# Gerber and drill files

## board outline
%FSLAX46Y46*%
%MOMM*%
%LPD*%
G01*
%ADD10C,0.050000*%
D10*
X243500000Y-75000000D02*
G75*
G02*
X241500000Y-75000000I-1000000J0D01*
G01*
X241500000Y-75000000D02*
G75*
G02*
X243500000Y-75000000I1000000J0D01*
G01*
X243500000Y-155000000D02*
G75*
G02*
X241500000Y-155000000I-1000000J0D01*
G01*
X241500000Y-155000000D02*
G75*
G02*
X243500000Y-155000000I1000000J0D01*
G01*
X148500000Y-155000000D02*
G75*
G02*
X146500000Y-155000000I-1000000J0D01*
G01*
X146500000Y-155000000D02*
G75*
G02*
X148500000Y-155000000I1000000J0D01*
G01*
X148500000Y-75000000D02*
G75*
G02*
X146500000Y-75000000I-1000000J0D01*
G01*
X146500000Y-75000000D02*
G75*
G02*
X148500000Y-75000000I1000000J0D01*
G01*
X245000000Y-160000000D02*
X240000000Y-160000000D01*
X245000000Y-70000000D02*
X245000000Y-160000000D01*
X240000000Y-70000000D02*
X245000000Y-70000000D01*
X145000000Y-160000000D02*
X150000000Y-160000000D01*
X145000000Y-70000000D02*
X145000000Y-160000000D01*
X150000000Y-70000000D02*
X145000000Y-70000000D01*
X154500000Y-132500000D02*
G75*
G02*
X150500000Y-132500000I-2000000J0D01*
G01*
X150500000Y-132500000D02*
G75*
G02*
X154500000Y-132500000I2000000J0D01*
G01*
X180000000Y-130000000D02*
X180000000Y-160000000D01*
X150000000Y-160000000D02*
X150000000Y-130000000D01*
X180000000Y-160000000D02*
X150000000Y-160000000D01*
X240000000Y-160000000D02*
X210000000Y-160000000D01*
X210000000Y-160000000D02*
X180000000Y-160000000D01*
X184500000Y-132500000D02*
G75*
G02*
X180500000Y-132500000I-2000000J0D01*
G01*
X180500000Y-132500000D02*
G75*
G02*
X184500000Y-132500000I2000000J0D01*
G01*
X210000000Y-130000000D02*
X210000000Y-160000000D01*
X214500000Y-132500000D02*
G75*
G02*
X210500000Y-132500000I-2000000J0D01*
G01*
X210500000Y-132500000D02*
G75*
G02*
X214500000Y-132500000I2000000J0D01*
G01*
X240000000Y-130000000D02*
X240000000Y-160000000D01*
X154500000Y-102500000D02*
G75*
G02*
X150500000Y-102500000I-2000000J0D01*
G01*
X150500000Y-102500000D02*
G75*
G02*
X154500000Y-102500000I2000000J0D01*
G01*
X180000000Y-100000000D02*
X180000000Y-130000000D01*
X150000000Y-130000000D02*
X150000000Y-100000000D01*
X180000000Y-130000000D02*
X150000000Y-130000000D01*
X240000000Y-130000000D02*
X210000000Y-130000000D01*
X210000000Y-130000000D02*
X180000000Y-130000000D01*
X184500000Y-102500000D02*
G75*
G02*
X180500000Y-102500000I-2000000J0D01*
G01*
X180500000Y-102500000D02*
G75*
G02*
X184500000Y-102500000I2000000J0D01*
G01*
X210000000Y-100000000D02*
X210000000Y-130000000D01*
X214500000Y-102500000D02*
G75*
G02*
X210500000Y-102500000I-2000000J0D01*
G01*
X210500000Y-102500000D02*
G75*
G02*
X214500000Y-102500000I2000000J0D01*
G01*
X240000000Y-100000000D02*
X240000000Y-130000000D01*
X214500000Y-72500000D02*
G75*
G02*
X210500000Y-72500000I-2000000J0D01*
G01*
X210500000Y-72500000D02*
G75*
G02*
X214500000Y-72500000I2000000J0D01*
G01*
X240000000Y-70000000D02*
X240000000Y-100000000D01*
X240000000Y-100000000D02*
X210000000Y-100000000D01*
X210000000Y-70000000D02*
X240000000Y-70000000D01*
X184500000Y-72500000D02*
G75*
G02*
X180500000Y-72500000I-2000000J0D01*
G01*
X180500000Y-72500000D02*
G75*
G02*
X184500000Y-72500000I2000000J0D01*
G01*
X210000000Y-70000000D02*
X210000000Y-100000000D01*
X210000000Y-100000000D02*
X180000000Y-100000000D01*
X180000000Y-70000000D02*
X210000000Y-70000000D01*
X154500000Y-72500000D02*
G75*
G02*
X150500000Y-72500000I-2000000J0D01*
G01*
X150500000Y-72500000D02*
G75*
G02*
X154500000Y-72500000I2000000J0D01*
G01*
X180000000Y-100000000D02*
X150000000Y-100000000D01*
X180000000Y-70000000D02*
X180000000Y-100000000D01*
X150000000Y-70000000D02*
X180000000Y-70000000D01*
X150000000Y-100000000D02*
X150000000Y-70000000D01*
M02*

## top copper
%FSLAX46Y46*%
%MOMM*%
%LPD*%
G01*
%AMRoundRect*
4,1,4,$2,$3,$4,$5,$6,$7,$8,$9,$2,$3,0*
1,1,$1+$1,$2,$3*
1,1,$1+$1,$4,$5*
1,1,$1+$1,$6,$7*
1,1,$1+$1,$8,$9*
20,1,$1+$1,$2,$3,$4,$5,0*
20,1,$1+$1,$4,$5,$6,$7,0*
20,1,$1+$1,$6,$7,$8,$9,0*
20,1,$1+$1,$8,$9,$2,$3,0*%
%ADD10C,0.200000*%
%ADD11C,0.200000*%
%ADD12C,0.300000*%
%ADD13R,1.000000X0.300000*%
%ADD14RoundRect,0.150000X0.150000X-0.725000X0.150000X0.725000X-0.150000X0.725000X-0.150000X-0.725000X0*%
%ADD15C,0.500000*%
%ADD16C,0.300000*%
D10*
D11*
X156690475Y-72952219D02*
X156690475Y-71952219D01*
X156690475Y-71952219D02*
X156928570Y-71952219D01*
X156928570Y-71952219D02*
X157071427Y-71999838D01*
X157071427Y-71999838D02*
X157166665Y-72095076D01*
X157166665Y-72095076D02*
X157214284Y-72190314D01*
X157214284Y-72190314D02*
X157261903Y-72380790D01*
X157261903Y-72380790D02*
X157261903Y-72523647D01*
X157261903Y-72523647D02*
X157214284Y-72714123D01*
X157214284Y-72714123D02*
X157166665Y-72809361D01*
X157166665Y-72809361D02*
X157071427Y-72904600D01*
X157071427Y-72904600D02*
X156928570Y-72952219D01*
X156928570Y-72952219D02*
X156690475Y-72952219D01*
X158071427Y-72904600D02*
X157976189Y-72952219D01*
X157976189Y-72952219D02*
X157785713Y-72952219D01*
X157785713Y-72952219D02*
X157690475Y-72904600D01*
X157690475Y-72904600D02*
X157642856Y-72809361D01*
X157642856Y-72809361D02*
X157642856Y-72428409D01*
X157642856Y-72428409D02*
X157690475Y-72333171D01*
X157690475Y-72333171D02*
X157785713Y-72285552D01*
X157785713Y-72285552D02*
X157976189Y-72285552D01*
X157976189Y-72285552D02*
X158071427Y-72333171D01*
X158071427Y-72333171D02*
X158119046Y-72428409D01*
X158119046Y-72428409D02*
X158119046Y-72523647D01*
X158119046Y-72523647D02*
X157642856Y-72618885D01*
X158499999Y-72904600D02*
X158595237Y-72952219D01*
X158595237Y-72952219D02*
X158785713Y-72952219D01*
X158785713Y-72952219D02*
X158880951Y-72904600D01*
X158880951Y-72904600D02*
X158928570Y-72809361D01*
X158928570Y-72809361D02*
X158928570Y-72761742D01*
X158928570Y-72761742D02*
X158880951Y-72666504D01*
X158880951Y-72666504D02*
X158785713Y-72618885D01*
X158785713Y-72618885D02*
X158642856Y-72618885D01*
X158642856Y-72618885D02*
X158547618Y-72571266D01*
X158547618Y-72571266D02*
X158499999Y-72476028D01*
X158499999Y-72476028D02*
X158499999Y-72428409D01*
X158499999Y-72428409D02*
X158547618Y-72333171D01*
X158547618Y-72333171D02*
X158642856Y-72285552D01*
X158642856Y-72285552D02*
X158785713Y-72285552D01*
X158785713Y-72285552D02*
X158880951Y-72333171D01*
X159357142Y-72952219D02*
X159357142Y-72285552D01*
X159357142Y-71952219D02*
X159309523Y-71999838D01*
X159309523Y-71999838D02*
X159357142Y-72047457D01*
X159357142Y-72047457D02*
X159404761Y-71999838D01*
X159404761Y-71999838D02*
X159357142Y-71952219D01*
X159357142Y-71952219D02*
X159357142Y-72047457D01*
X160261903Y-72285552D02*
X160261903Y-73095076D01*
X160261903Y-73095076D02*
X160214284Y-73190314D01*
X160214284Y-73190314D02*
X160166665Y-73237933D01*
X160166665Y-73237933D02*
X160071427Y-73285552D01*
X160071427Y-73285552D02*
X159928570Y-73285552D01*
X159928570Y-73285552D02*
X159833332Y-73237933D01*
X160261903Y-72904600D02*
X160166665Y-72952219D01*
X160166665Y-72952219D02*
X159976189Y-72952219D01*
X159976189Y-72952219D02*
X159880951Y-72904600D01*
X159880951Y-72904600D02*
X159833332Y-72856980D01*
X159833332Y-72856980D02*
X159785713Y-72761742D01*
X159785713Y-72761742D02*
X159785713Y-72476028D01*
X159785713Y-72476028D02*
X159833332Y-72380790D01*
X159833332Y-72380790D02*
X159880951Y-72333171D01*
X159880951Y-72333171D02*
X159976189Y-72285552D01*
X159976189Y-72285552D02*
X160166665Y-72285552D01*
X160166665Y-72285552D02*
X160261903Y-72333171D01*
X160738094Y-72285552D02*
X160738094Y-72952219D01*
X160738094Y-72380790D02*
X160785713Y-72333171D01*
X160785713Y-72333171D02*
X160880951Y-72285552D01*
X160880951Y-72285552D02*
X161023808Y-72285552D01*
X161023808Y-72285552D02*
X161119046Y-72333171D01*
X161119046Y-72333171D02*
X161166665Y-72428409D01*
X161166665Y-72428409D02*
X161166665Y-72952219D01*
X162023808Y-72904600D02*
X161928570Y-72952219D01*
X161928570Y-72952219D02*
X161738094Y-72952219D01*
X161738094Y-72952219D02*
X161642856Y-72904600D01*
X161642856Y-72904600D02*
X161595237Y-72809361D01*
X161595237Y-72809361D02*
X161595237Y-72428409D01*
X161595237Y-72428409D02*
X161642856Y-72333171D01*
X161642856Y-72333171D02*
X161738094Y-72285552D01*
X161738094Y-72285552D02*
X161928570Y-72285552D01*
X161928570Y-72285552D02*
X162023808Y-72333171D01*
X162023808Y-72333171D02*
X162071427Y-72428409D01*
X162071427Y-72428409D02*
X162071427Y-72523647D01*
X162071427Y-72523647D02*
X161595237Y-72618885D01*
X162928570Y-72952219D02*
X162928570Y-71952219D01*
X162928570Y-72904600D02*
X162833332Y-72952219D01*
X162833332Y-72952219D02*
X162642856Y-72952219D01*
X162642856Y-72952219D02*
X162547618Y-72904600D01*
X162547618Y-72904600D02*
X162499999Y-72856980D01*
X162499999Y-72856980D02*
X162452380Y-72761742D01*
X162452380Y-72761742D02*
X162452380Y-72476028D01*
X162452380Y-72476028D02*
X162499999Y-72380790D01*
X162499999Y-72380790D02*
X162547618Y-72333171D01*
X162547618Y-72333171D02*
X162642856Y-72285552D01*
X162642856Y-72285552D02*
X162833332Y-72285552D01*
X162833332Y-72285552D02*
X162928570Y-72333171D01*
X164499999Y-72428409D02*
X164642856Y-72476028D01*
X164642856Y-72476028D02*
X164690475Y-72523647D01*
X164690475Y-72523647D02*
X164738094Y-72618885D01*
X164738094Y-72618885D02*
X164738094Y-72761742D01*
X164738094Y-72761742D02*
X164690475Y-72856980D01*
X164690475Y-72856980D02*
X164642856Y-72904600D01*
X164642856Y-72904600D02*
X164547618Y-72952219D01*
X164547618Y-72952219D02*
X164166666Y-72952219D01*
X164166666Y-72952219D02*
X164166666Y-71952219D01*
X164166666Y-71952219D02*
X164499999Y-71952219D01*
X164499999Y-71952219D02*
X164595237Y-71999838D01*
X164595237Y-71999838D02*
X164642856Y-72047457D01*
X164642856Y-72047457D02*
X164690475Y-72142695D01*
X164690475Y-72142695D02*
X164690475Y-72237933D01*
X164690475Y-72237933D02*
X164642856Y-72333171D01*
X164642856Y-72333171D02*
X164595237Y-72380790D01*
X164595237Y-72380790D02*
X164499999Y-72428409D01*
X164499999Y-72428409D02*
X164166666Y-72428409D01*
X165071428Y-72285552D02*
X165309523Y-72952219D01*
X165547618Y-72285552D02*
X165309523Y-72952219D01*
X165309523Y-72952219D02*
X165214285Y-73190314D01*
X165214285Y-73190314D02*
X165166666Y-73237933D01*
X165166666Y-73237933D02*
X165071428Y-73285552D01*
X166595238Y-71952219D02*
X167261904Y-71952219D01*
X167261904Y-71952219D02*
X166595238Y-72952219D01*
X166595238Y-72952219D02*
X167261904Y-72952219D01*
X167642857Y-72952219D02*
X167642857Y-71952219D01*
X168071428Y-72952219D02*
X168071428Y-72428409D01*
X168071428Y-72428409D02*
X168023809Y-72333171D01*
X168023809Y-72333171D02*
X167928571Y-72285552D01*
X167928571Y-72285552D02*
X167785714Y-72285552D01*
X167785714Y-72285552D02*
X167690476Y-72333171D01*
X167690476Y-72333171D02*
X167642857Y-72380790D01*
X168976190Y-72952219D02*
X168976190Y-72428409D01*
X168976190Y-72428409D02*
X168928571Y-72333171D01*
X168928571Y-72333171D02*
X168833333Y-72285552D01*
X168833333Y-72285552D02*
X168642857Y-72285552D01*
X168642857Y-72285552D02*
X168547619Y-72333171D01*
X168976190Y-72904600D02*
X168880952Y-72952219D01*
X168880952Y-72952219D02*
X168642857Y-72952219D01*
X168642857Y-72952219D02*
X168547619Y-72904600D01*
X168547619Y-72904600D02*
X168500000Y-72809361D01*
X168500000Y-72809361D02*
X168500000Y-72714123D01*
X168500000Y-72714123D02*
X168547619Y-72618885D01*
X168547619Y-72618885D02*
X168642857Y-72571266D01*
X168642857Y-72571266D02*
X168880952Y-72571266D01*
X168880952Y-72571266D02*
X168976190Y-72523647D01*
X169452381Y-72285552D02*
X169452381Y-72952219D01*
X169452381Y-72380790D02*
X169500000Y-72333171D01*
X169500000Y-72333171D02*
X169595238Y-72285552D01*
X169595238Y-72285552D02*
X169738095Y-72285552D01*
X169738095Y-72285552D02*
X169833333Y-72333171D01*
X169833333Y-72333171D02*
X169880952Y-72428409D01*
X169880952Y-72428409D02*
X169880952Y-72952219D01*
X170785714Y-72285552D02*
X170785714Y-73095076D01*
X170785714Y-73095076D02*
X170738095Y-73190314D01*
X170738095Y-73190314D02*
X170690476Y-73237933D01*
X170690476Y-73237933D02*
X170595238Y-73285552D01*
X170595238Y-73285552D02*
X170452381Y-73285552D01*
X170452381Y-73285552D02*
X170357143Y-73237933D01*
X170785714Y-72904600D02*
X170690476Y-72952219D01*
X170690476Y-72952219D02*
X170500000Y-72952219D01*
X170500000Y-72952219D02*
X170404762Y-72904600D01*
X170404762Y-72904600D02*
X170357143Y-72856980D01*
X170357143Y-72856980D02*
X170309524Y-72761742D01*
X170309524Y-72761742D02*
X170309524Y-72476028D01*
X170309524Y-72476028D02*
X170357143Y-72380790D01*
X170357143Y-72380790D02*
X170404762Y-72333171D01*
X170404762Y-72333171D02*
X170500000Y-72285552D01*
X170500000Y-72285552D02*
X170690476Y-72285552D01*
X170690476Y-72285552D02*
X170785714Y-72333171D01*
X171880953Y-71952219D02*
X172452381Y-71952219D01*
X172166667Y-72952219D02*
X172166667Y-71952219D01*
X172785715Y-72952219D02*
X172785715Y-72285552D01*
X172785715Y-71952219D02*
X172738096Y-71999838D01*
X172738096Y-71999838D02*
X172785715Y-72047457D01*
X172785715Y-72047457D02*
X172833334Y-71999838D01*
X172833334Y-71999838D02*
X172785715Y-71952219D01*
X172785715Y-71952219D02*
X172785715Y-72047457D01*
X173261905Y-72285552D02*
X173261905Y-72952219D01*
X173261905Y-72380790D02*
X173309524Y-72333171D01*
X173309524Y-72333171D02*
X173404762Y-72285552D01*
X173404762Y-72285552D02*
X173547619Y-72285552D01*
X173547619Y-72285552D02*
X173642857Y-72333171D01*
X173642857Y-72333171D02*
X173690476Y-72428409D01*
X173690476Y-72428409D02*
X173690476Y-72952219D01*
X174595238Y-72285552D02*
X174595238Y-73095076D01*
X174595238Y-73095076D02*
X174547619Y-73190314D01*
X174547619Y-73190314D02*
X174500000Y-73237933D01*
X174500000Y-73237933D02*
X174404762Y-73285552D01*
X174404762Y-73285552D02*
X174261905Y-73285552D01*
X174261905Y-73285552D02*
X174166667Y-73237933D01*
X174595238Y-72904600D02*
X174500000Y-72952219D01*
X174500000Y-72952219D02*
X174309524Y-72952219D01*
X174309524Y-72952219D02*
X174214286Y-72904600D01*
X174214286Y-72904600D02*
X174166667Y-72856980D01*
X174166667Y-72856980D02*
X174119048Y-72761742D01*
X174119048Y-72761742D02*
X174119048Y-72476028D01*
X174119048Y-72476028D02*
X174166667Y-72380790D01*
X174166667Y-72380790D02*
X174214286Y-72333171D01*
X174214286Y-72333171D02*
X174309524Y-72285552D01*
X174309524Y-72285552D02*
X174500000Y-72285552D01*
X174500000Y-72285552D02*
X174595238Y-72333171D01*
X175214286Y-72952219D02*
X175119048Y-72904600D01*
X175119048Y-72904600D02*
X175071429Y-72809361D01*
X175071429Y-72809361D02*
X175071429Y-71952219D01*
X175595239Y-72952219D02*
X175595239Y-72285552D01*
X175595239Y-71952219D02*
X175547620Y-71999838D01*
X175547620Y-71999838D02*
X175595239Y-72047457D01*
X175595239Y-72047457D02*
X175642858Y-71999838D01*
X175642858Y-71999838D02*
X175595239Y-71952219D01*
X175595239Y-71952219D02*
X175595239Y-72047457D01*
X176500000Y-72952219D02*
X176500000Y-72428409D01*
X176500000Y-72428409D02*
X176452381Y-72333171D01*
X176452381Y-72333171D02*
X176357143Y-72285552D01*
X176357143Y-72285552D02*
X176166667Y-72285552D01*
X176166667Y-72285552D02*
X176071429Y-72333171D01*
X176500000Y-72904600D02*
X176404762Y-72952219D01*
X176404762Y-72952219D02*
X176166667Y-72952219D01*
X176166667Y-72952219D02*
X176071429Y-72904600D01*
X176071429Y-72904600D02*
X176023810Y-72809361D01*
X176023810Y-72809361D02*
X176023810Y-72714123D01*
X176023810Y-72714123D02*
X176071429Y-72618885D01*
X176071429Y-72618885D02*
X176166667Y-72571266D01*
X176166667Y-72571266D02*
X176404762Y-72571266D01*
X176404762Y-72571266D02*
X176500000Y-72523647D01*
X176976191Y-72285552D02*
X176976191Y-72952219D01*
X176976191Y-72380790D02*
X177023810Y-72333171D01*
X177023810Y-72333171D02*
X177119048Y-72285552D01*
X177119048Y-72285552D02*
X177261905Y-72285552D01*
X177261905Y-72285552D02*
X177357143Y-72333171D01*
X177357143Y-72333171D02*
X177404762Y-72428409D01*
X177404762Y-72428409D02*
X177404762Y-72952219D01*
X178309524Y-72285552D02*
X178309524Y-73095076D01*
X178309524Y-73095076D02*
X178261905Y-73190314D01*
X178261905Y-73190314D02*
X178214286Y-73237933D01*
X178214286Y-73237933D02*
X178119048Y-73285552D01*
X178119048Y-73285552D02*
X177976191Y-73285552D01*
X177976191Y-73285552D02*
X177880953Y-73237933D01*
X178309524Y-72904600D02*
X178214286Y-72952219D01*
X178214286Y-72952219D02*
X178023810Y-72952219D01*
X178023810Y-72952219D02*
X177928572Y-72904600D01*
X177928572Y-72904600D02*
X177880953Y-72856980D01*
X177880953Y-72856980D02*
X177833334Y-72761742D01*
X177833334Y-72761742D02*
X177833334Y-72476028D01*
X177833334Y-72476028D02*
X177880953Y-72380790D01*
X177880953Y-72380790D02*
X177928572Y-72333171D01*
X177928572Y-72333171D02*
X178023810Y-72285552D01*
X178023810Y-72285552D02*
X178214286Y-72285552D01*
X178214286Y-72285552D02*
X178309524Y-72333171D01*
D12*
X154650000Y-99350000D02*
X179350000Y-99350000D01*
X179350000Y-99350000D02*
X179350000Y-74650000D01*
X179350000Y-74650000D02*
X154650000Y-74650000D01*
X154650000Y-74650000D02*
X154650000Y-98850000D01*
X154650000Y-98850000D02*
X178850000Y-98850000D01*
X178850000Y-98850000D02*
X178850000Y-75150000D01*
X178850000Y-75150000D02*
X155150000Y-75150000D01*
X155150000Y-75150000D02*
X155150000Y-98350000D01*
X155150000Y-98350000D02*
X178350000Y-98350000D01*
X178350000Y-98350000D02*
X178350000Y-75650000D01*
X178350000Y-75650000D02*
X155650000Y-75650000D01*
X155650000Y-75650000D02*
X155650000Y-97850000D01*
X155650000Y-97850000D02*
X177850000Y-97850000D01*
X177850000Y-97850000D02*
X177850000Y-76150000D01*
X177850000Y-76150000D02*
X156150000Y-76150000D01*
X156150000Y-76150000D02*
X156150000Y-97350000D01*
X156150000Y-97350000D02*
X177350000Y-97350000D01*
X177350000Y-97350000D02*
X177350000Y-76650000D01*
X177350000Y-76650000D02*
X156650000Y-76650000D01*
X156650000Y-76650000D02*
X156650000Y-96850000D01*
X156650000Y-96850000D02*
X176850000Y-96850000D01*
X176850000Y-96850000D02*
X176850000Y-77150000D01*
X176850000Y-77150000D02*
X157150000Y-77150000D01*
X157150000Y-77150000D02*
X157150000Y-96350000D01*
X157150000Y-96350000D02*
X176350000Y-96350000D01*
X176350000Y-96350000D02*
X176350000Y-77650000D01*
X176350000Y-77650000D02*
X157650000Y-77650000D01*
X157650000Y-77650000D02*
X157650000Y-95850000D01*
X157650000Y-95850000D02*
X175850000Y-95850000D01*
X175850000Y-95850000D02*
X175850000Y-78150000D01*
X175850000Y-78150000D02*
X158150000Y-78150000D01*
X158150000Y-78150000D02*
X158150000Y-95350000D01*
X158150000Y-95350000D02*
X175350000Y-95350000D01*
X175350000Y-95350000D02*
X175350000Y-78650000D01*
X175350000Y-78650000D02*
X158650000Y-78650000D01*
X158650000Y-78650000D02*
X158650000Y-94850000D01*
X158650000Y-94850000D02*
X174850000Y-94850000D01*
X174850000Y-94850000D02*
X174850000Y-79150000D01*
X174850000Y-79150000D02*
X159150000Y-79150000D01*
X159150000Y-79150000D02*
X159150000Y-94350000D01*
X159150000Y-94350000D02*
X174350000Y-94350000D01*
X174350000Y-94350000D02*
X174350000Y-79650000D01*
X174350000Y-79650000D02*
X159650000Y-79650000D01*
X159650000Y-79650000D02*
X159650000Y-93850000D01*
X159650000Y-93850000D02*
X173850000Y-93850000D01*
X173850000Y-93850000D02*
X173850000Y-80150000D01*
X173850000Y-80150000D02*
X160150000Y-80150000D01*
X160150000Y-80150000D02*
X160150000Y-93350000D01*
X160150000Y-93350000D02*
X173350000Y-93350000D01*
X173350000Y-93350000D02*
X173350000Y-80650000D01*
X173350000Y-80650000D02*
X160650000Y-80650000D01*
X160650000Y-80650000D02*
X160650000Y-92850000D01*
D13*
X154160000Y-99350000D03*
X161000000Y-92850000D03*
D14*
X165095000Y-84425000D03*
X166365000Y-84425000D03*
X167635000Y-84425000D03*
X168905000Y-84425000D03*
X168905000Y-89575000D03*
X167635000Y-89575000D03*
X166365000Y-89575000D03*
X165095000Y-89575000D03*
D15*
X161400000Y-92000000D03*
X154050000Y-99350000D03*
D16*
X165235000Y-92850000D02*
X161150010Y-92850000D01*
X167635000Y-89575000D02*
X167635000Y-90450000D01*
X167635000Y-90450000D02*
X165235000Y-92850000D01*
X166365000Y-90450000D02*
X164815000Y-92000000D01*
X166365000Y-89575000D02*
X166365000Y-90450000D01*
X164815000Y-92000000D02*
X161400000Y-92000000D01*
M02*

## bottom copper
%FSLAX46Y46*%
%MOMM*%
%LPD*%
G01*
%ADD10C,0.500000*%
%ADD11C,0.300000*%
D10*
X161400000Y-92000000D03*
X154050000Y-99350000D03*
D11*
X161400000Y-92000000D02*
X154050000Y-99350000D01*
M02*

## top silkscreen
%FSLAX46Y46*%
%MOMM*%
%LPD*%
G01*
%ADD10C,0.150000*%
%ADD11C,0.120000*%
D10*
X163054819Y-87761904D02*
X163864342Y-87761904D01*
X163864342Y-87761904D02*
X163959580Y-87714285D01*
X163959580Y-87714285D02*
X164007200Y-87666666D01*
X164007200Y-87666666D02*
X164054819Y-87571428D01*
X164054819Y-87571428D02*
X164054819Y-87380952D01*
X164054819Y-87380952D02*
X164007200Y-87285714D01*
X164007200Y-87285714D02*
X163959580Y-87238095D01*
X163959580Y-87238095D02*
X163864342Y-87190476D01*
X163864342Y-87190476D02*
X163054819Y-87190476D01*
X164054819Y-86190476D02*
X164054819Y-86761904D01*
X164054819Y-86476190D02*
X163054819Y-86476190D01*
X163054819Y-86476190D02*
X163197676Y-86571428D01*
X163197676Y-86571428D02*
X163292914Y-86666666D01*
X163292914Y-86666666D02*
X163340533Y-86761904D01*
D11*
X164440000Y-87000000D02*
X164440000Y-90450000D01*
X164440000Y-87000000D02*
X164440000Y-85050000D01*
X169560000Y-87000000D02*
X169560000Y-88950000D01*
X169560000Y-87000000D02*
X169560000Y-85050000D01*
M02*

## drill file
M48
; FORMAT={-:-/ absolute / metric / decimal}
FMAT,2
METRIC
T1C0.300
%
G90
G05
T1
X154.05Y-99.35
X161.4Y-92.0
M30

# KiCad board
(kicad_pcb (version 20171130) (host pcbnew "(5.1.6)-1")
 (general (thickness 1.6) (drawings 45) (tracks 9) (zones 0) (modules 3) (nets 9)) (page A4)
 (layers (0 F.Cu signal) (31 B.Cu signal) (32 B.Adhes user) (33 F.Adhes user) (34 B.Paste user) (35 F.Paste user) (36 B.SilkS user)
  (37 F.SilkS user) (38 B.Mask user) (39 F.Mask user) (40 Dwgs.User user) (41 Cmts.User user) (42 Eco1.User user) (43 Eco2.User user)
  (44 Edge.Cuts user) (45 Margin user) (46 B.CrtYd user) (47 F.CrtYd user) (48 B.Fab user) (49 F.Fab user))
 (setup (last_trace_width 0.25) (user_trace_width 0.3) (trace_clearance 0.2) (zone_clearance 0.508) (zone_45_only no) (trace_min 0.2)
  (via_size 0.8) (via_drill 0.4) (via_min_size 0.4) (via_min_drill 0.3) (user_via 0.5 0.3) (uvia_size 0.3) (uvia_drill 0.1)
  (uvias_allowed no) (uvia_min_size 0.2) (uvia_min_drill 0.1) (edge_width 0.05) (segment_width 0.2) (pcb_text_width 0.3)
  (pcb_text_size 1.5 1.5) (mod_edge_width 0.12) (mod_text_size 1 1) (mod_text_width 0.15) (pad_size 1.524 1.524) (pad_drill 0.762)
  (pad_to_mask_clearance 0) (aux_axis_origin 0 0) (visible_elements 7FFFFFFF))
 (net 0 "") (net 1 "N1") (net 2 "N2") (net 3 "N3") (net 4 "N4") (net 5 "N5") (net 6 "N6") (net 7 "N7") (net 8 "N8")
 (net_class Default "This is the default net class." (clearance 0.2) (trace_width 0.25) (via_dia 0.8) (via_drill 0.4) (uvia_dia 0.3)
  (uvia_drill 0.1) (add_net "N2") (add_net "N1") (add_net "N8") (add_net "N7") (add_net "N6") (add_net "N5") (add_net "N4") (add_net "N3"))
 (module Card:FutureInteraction (layer B.Cu) (at 165 82.5 180)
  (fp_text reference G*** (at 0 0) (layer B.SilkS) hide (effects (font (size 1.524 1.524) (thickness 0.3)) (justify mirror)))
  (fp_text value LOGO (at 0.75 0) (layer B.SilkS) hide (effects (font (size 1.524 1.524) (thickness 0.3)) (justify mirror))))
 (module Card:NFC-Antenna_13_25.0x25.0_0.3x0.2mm (layer F.Cu) (at 167 87)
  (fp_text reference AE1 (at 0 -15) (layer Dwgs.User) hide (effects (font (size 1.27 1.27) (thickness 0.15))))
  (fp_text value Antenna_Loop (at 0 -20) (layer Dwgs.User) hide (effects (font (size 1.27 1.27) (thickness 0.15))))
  (fp_line (start -12.35 12.35) (end 12.35 12.35) (layer F.Cu) (width 0.3))
  (fp_line (start 12.35 12.35) (end 12.35 -12.35) (layer F.Cu) (width 0.3))
  (fp_line (start 12.35 -12.35) (end -12.35 -12.35) (layer F.Cu) (width 0.3))
  (fp_line (start -12.35 -12.35) (end -12.35 11.85) (layer F.Cu) (width 0.3))
  (fp_line (start -12.35 11.85) (end 11.85 11.85) (layer F.Cu) (width 0.3))
  (fp_line (start 11.85 11.85) (end 11.85 -11.85) (layer F.Cu) (width 0.3))
  (fp_line (start 11.85 -11.85) (end -11.85 -11.85) (layer F.Cu) (width 0.3))
  (fp_line (start -11.85 -11.85) (end -11.85 11.35) (layer F.Cu) (width 0.3))
  (fp_line (start -11.85 11.35) (end 11.35 11.35) (layer F.Cu) (width 0.3))
  (fp_line (start 11.35 11.35) (end 11.35 -11.35) (layer F.Cu) (width 0.3))
  (fp_line (start 11.35 -11.35) (end -11.35 -11.35) (layer F.Cu) (width 0.3))
  (fp_line (start -11.35 -11.35) (end -11.35 10.85) (layer F.Cu) (width 0.3))
  (fp_line (start -11.35 10.85) (end 10.85 10.85) (layer F.Cu) (width 0.3))
  (fp_line (start 10.85 10.85) (end 10.85 -10.85) (layer F.Cu) (width 0.3))
  (fp_line (start 10.85 -10.85) (end -10.85 -10.85) (layer F.Cu) (width 0.3))
  (fp_line (start -10.85 -10.85) (end -10.85 10.35) (layer F.Cu) (width 0.3))
  (fp_line (start -10.85 10.35) (end 10.35 10.35) (layer F.Cu) (width 0.3))
  (fp_line (start 10.35 10.35) (end 10.35 -10.35) (layer F.Cu) (width 0.3))
  (fp_line (start 10.35 -10.35) (end -10.35 -10.35) (layer F.Cu) (width 0.3))
  (fp_line (start -10.35 -10.35) (end -10.35 9.85) (layer F.Cu) (width 0.3))
  (fp_line (start -10.35 9.85) (end 9.85 9.85) (layer F.Cu) (width 0.3))
  (fp_line (start 9.85 9.85) (end 9.85 -9.85) (layer F.Cu) (width 0.3))
  (fp_line (start 9.85 -9.85) (end -9.85 -9.85) (layer F.Cu) (width 0.3))
  (fp_line (start -9.85 -9.85) (end -9.85 9.35) (layer F.Cu) (width 0.3))
  (fp_line (start -9.85 9.35) (end 9.35 9.35) (layer F.Cu) (width 0.3))
  (fp_line (start 9.35 9.35) (end 9.35 -9.35) (layer F.Cu) (width 0.3))
  (fp_line (start 9.35 -9.35) (end -9.35 -9.35) (layer F.Cu) (width 0.3))
  (fp_line (start -9.35 -9.35) (end -9.35 8.85) (layer F.Cu) (width 0.3))
  (fp_line (start -9.35 8.85) (end 8.85 8.85) (layer F.Cu) (width 0.3))
  (fp_line (start 8.85 8.85) (end 8.85 -8.85) (layer F.Cu) (width 0.3))
  (fp_line (start 8.85 -8.85) (end -8.85 -8.85) (layer F.Cu) (width 0.3))
  (fp_line (start -8.85 -8.85) (end -8.85 8.35) (layer F.Cu) (width 0.3))
  (fp_line (start -8.85 8.35) (end 8.35 8.35) (layer F.Cu) (width 0.3))
  (fp_line (start 8.35 8.35) (end 8.35 -8.35) (layer F.Cu) (width 0.3))
  (fp_line (start 8.35 -8.35) (end -8.35 -8.35) (layer F.Cu) (width 0.3))
  (fp_line (start -8.35 -8.35) (end -8.35 7.85) (layer F.Cu) (width 0.3))
  (fp_line (start -8.35 7.85) (end 7.85 7.85) (layer F.Cu) (width 0.3))
  (fp_line (start 7.85 7.85) (end 7.85 -7.85) (layer F.Cu) (width 0.3))
  (fp_line (start 7.85 -7.85) (end -7.85 -7.85) (layer F.Cu) (width 0.3))
  (fp_line (start -7.85 -7.85) (end -7.85 7.35) (layer F.Cu) (width 0.3))
  (fp_line (start -7.85 7.35) (end 7.35 7.35) (layer F.Cu) (width 0.3))
  (fp_line (start 7.35 7.35) (end 7.35 -7.35) (layer F.Cu) (width 0.3))
  (fp_line (start 7.35 -7.35) (end -7.35 -7.35) (layer F.Cu) (width 0.3))
  (fp_line (start -7.35 -7.35) (end -7.35 6.85) (layer F.Cu) (width 0.3))
  (fp_line (start -7.35 6.85) (end 6.85 6.85) (layer F.Cu) (width 0.3))
  (fp_line (start 6.85 6.85) (end 6.85 -6.85) (layer F.Cu) (width 0.3))
  (fp_line (start 6.85 -6.85) (end -6.85 -6.85) (layer F.Cu) (width 0.3))
  (fp_line (start -6.85 -6.85) (end -6.85 6.35) (layer F.Cu) (width 0.3))
  (fp_line (start -6.85 6.35) (end 6.35 6.35) (layer F.Cu) (width 0.3))
  (fp_line (start 6.35 6.35) (end 6.35 -6.35) (layer F.Cu) (width 0.3))
  (fp_line (start 6.35 -6.35) (end -6.35 -6.35) (layer F.Cu) (width 0.3))
  (fp_line (start -6.35 -6.35) (end -6.35 5.85) (layer F.Cu) (width 0.3))
  (pad 2 smd rect (at -12.84 12.35) (size 1 0.3) (layers F.Cu) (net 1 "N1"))
  (pad 1 smd rect (at -6 5.85) (size 1 0.3) (layers F.Cu) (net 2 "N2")))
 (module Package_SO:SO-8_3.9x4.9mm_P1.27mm (layer F.Cu) (at 167 87 90)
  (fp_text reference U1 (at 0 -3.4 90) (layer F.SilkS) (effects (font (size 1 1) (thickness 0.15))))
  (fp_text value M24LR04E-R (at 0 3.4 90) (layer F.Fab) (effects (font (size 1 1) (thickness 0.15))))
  (fp_line (start 0 -2.56) (end -3.45 -2.56) (layer F.SilkS) (width 0.12))
  (fp_line (start 0 -2.56) (end 1.95 -2.56) (layer F.SilkS) (width 0.12))
  (fp_line (start 0 2.56) (end -1.95 2.56) (layer F.SilkS) (width 0.12))
  (fp_line (start 0 2.56) (end 1.95 2.56) (layer F.SilkS) (width 0.12))
  (pad 8 smd roundrect (at 2.575 -1.905 90) (size 1.75 0.6) (layers F.Cu F.Paste F.Mask) (roundrect_rratio 0.25) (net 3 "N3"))
  (pad 7 smd roundrect (at 2.575 -0.635 90) (size 1.75 0.6) (layers F.Cu F.Paste F.Mask) (roundrect_rratio 0.25) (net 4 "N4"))
  (pad 6 smd roundrect (at 2.575 0.635 90) (size 1.75 0.6) (layers F.Cu F.Paste F.Mask) (roundrect_rratio 0.25) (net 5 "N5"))
  (pad 5 smd roundrect (at 2.575 1.905 90) (size 1.75 0.6) (layers F.Cu F.Paste F.Mask) (roundrect_rratio 0.25) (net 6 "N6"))
  (pad 4 smd roundrect (at -2.575 1.905 90) (size 1.75 0.6) (layers F.Cu F.Paste F.Mask) (roundrect_rratio 0.25) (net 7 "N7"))
  (pad 3 smd roundrect (at -2.575 0.635 90) (size 1.75 0.6) (layers F.Cu F.Paste F.Mask) (roundrect_rratio 0.25) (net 2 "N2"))
  (pad 2 smd roundrect (at -2.575 -0.635 90) (size 1.75 0.6) (layers F.Cu F.Paste F.Mask) (roundrect_rratio 0.25) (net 1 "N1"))
  (pad 1 smd roundrect (at -2.575 -1.905 90) (size 1.75 0.6) (layers F.Cu F.Paste F.Mask) (roundrect_rratio 0.25) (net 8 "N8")))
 (gr_circle (center 242.5 75) (end 243.5 75) (layer Edge.Cuts) (width 0.05))
 (gr_circle (center 242.5 155) (end 243.5 155) (layer Edge.Cuts) (width 0.05))
 (gr_circle (center 147.5 155) (end 148.5 155) (layer Edge.Cuts) (width 0.05))
 (gr_circle (center 147.5 75) (end 148.5 75) (layer Edge.Cuts) (width 0.05))
 (gr_line (start 245 160) (end 240 160) (layer Edge.Cuts) (width 0.05))
 (gr_line (start 245 70) (end 245 160) (layer Edge.Cuts) (width 0.05))
 (gr_line (start 240 70) (end 245 70) (layer Edge.Cuts) (width 0.05))
 (gr_line (start 145 160) (end 150 160) (layer Edge.Cuts) (width 0.05))
 (gr_line (start 145 70) (end 145 160) (layer Edge.Cuts) (width 0.05))
 (gr_line (start 150 70) (end 145 70) (layer Edge.Cuts) (width 0.05))
 (gr_circle (center 152.5 132.5) (end 154.5 132.5) (layer Edge.Cuts) (width 0.05))
 (gr_line (start 180 130) (end 180 160) (layer Edge.Cuts) (width 0.05))
 (gr_line (start 150 160) (end 150 130) (layer Edge.Cuts) (width 0.05))
 (gr_line (start 180 160) (end 150 160) (layer Edge.Cuts) (width 0.05))
 (gr_line (start 240 160) (end 210 160) (layer Edge.Cuts) (width 0.05))
 (gr_line (start 210 160) (end 180 160) (layer Edge.Cuts) (width 0.05))
 (gr_circle (center 182.5 132.5) (end 184.5 132.5) (layer Edge.Cuts) (width 0.05))
 (gr_line (start 210 130) (end 210 160) (layer Edge.Cuts) (width 0.05))
 (gr_circle (center 212.5 132.5) (end 214.5 132.5) (layer Edge.Cuts) (width 0.05))
 (gr_line (start 240 130) (end 240 160) (layer Edge.Cuts) (width 0.05))
 (gr_circle (center 152.5 102.5) (end 154.5 102.5) (layer Edge.Cuts) (width 0.05))
 (gr_line (start 180 100) (end 180 130) (layer Edge.Cuts) (width 0.05))
 (gr_line (start 150 130) (end 150 100) (layer Edge.Cuts) (width 0.05))
 (gr_line (start 180 130) (end 150 130) (layer Edge.Cuts) (width 0.05))
 (gr_line (start 240 130) (end 210 130) (layer Edge.Cuts) (width 0.05))
 (gr_line (start 210 130) (end 180 130) (layer Edge.Cuts) (width 0.05))
 (gr_circle (center 182.5 102.5) (end 184.5 102.5) (layer Edge.Cuts) (width 0.05))
 (gr_line (start 210 100) (end 210 130) (layer Edge.Cuts) (width 0.05))
 (gr_circle (center 212.5 102.5) (end 214.5 102.5) (layer Edge.Cuts) (width 0.05))
 (gr_line (start 240 100) (end 240 130) (layer Edge.Cuts) (width 0.05))
 (gr_circle (center 212.5 72.5) (end 214.5 72.5) (layer Edge.Cuts) (width 0.05))
 (gr_line (start 240 70) (end 240 100) (layer Edge.Cuts) (width 0.05))
 (gr_line (start 240 100) (end 210 100) (layer Edge.Cuts) (width 0.05))
 (gr_line (start 210 70) (end 240 70) (layer Edge.Cuts) (width 0.05))
 (gr_circle (center 182.5 72.5) (end 184.5 72.5) (layer Edge.Cuts) (width 0.05))
 (gr_line (start 210 70) (end 210 100) (layer Edge.Cuts) (width 0.05))
 (gr_line (start 210 100) (end 180 100) (layer Edge.Cuts) (width 0.05))
 (gr_line (start 180 70) (end 210 70) (layer Edge.Cuts) (width 0.05))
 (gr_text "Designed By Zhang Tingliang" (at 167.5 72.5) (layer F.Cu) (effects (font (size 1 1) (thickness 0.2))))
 (gr_circle (center 152.5 72.5) (end 154.5 72.5) (layer Edge.Cuts) (width 0.05))
 (gr_line (start 180 100) (end 150 100) (layer Edge.Cuts) (width 0.05))
 (gr_line (start 180 70) (end 180 100) (layer Edge.Cuts) (width 0.05))
 (gr_line (start 150 70) (end 180 70) (layer Edge.Cuts) (width 0.05))
 (gr_line (start 150 100) (end 150 70) (layer Edge.Cuts) (width 0.05))
 (segment (start 165.235 92.85) (end 161.15001 92.85) (width 0.3) (layer F.Cu) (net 2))
 (segment (start 167.635 89.575) (end 167.635 90.45) (width 0.3) (layer F.Cu) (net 2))
 (segment (start 167.635 90.45) (end 165.235 92.85) (width 0.3) (layer F.Cu) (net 2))
 (segment (start 166.365 90.45) (end 164.815 92) (width 0.3) (layer F.Cu) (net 1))
 (segment (start 166.365 89.575) (end 166.365 90.45) (width 0.3) (layer F.Cu) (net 1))
 (via (at 161.4 92) (size 0.5) (drill 0.3) (layers F.Cu B.Cu) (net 1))
 (segment (start 164.815 92) (end 161.4 92) (width 0.3) (layer F.Cu) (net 1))
 (via (at 154.05 99.35) (size 0.5) (drill 0.3) (layers F.Cu B.Cu) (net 1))
 (segment (start 161.4 92) (end 154.05 99.35) (width 0.3) (layer B.Cu) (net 1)))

